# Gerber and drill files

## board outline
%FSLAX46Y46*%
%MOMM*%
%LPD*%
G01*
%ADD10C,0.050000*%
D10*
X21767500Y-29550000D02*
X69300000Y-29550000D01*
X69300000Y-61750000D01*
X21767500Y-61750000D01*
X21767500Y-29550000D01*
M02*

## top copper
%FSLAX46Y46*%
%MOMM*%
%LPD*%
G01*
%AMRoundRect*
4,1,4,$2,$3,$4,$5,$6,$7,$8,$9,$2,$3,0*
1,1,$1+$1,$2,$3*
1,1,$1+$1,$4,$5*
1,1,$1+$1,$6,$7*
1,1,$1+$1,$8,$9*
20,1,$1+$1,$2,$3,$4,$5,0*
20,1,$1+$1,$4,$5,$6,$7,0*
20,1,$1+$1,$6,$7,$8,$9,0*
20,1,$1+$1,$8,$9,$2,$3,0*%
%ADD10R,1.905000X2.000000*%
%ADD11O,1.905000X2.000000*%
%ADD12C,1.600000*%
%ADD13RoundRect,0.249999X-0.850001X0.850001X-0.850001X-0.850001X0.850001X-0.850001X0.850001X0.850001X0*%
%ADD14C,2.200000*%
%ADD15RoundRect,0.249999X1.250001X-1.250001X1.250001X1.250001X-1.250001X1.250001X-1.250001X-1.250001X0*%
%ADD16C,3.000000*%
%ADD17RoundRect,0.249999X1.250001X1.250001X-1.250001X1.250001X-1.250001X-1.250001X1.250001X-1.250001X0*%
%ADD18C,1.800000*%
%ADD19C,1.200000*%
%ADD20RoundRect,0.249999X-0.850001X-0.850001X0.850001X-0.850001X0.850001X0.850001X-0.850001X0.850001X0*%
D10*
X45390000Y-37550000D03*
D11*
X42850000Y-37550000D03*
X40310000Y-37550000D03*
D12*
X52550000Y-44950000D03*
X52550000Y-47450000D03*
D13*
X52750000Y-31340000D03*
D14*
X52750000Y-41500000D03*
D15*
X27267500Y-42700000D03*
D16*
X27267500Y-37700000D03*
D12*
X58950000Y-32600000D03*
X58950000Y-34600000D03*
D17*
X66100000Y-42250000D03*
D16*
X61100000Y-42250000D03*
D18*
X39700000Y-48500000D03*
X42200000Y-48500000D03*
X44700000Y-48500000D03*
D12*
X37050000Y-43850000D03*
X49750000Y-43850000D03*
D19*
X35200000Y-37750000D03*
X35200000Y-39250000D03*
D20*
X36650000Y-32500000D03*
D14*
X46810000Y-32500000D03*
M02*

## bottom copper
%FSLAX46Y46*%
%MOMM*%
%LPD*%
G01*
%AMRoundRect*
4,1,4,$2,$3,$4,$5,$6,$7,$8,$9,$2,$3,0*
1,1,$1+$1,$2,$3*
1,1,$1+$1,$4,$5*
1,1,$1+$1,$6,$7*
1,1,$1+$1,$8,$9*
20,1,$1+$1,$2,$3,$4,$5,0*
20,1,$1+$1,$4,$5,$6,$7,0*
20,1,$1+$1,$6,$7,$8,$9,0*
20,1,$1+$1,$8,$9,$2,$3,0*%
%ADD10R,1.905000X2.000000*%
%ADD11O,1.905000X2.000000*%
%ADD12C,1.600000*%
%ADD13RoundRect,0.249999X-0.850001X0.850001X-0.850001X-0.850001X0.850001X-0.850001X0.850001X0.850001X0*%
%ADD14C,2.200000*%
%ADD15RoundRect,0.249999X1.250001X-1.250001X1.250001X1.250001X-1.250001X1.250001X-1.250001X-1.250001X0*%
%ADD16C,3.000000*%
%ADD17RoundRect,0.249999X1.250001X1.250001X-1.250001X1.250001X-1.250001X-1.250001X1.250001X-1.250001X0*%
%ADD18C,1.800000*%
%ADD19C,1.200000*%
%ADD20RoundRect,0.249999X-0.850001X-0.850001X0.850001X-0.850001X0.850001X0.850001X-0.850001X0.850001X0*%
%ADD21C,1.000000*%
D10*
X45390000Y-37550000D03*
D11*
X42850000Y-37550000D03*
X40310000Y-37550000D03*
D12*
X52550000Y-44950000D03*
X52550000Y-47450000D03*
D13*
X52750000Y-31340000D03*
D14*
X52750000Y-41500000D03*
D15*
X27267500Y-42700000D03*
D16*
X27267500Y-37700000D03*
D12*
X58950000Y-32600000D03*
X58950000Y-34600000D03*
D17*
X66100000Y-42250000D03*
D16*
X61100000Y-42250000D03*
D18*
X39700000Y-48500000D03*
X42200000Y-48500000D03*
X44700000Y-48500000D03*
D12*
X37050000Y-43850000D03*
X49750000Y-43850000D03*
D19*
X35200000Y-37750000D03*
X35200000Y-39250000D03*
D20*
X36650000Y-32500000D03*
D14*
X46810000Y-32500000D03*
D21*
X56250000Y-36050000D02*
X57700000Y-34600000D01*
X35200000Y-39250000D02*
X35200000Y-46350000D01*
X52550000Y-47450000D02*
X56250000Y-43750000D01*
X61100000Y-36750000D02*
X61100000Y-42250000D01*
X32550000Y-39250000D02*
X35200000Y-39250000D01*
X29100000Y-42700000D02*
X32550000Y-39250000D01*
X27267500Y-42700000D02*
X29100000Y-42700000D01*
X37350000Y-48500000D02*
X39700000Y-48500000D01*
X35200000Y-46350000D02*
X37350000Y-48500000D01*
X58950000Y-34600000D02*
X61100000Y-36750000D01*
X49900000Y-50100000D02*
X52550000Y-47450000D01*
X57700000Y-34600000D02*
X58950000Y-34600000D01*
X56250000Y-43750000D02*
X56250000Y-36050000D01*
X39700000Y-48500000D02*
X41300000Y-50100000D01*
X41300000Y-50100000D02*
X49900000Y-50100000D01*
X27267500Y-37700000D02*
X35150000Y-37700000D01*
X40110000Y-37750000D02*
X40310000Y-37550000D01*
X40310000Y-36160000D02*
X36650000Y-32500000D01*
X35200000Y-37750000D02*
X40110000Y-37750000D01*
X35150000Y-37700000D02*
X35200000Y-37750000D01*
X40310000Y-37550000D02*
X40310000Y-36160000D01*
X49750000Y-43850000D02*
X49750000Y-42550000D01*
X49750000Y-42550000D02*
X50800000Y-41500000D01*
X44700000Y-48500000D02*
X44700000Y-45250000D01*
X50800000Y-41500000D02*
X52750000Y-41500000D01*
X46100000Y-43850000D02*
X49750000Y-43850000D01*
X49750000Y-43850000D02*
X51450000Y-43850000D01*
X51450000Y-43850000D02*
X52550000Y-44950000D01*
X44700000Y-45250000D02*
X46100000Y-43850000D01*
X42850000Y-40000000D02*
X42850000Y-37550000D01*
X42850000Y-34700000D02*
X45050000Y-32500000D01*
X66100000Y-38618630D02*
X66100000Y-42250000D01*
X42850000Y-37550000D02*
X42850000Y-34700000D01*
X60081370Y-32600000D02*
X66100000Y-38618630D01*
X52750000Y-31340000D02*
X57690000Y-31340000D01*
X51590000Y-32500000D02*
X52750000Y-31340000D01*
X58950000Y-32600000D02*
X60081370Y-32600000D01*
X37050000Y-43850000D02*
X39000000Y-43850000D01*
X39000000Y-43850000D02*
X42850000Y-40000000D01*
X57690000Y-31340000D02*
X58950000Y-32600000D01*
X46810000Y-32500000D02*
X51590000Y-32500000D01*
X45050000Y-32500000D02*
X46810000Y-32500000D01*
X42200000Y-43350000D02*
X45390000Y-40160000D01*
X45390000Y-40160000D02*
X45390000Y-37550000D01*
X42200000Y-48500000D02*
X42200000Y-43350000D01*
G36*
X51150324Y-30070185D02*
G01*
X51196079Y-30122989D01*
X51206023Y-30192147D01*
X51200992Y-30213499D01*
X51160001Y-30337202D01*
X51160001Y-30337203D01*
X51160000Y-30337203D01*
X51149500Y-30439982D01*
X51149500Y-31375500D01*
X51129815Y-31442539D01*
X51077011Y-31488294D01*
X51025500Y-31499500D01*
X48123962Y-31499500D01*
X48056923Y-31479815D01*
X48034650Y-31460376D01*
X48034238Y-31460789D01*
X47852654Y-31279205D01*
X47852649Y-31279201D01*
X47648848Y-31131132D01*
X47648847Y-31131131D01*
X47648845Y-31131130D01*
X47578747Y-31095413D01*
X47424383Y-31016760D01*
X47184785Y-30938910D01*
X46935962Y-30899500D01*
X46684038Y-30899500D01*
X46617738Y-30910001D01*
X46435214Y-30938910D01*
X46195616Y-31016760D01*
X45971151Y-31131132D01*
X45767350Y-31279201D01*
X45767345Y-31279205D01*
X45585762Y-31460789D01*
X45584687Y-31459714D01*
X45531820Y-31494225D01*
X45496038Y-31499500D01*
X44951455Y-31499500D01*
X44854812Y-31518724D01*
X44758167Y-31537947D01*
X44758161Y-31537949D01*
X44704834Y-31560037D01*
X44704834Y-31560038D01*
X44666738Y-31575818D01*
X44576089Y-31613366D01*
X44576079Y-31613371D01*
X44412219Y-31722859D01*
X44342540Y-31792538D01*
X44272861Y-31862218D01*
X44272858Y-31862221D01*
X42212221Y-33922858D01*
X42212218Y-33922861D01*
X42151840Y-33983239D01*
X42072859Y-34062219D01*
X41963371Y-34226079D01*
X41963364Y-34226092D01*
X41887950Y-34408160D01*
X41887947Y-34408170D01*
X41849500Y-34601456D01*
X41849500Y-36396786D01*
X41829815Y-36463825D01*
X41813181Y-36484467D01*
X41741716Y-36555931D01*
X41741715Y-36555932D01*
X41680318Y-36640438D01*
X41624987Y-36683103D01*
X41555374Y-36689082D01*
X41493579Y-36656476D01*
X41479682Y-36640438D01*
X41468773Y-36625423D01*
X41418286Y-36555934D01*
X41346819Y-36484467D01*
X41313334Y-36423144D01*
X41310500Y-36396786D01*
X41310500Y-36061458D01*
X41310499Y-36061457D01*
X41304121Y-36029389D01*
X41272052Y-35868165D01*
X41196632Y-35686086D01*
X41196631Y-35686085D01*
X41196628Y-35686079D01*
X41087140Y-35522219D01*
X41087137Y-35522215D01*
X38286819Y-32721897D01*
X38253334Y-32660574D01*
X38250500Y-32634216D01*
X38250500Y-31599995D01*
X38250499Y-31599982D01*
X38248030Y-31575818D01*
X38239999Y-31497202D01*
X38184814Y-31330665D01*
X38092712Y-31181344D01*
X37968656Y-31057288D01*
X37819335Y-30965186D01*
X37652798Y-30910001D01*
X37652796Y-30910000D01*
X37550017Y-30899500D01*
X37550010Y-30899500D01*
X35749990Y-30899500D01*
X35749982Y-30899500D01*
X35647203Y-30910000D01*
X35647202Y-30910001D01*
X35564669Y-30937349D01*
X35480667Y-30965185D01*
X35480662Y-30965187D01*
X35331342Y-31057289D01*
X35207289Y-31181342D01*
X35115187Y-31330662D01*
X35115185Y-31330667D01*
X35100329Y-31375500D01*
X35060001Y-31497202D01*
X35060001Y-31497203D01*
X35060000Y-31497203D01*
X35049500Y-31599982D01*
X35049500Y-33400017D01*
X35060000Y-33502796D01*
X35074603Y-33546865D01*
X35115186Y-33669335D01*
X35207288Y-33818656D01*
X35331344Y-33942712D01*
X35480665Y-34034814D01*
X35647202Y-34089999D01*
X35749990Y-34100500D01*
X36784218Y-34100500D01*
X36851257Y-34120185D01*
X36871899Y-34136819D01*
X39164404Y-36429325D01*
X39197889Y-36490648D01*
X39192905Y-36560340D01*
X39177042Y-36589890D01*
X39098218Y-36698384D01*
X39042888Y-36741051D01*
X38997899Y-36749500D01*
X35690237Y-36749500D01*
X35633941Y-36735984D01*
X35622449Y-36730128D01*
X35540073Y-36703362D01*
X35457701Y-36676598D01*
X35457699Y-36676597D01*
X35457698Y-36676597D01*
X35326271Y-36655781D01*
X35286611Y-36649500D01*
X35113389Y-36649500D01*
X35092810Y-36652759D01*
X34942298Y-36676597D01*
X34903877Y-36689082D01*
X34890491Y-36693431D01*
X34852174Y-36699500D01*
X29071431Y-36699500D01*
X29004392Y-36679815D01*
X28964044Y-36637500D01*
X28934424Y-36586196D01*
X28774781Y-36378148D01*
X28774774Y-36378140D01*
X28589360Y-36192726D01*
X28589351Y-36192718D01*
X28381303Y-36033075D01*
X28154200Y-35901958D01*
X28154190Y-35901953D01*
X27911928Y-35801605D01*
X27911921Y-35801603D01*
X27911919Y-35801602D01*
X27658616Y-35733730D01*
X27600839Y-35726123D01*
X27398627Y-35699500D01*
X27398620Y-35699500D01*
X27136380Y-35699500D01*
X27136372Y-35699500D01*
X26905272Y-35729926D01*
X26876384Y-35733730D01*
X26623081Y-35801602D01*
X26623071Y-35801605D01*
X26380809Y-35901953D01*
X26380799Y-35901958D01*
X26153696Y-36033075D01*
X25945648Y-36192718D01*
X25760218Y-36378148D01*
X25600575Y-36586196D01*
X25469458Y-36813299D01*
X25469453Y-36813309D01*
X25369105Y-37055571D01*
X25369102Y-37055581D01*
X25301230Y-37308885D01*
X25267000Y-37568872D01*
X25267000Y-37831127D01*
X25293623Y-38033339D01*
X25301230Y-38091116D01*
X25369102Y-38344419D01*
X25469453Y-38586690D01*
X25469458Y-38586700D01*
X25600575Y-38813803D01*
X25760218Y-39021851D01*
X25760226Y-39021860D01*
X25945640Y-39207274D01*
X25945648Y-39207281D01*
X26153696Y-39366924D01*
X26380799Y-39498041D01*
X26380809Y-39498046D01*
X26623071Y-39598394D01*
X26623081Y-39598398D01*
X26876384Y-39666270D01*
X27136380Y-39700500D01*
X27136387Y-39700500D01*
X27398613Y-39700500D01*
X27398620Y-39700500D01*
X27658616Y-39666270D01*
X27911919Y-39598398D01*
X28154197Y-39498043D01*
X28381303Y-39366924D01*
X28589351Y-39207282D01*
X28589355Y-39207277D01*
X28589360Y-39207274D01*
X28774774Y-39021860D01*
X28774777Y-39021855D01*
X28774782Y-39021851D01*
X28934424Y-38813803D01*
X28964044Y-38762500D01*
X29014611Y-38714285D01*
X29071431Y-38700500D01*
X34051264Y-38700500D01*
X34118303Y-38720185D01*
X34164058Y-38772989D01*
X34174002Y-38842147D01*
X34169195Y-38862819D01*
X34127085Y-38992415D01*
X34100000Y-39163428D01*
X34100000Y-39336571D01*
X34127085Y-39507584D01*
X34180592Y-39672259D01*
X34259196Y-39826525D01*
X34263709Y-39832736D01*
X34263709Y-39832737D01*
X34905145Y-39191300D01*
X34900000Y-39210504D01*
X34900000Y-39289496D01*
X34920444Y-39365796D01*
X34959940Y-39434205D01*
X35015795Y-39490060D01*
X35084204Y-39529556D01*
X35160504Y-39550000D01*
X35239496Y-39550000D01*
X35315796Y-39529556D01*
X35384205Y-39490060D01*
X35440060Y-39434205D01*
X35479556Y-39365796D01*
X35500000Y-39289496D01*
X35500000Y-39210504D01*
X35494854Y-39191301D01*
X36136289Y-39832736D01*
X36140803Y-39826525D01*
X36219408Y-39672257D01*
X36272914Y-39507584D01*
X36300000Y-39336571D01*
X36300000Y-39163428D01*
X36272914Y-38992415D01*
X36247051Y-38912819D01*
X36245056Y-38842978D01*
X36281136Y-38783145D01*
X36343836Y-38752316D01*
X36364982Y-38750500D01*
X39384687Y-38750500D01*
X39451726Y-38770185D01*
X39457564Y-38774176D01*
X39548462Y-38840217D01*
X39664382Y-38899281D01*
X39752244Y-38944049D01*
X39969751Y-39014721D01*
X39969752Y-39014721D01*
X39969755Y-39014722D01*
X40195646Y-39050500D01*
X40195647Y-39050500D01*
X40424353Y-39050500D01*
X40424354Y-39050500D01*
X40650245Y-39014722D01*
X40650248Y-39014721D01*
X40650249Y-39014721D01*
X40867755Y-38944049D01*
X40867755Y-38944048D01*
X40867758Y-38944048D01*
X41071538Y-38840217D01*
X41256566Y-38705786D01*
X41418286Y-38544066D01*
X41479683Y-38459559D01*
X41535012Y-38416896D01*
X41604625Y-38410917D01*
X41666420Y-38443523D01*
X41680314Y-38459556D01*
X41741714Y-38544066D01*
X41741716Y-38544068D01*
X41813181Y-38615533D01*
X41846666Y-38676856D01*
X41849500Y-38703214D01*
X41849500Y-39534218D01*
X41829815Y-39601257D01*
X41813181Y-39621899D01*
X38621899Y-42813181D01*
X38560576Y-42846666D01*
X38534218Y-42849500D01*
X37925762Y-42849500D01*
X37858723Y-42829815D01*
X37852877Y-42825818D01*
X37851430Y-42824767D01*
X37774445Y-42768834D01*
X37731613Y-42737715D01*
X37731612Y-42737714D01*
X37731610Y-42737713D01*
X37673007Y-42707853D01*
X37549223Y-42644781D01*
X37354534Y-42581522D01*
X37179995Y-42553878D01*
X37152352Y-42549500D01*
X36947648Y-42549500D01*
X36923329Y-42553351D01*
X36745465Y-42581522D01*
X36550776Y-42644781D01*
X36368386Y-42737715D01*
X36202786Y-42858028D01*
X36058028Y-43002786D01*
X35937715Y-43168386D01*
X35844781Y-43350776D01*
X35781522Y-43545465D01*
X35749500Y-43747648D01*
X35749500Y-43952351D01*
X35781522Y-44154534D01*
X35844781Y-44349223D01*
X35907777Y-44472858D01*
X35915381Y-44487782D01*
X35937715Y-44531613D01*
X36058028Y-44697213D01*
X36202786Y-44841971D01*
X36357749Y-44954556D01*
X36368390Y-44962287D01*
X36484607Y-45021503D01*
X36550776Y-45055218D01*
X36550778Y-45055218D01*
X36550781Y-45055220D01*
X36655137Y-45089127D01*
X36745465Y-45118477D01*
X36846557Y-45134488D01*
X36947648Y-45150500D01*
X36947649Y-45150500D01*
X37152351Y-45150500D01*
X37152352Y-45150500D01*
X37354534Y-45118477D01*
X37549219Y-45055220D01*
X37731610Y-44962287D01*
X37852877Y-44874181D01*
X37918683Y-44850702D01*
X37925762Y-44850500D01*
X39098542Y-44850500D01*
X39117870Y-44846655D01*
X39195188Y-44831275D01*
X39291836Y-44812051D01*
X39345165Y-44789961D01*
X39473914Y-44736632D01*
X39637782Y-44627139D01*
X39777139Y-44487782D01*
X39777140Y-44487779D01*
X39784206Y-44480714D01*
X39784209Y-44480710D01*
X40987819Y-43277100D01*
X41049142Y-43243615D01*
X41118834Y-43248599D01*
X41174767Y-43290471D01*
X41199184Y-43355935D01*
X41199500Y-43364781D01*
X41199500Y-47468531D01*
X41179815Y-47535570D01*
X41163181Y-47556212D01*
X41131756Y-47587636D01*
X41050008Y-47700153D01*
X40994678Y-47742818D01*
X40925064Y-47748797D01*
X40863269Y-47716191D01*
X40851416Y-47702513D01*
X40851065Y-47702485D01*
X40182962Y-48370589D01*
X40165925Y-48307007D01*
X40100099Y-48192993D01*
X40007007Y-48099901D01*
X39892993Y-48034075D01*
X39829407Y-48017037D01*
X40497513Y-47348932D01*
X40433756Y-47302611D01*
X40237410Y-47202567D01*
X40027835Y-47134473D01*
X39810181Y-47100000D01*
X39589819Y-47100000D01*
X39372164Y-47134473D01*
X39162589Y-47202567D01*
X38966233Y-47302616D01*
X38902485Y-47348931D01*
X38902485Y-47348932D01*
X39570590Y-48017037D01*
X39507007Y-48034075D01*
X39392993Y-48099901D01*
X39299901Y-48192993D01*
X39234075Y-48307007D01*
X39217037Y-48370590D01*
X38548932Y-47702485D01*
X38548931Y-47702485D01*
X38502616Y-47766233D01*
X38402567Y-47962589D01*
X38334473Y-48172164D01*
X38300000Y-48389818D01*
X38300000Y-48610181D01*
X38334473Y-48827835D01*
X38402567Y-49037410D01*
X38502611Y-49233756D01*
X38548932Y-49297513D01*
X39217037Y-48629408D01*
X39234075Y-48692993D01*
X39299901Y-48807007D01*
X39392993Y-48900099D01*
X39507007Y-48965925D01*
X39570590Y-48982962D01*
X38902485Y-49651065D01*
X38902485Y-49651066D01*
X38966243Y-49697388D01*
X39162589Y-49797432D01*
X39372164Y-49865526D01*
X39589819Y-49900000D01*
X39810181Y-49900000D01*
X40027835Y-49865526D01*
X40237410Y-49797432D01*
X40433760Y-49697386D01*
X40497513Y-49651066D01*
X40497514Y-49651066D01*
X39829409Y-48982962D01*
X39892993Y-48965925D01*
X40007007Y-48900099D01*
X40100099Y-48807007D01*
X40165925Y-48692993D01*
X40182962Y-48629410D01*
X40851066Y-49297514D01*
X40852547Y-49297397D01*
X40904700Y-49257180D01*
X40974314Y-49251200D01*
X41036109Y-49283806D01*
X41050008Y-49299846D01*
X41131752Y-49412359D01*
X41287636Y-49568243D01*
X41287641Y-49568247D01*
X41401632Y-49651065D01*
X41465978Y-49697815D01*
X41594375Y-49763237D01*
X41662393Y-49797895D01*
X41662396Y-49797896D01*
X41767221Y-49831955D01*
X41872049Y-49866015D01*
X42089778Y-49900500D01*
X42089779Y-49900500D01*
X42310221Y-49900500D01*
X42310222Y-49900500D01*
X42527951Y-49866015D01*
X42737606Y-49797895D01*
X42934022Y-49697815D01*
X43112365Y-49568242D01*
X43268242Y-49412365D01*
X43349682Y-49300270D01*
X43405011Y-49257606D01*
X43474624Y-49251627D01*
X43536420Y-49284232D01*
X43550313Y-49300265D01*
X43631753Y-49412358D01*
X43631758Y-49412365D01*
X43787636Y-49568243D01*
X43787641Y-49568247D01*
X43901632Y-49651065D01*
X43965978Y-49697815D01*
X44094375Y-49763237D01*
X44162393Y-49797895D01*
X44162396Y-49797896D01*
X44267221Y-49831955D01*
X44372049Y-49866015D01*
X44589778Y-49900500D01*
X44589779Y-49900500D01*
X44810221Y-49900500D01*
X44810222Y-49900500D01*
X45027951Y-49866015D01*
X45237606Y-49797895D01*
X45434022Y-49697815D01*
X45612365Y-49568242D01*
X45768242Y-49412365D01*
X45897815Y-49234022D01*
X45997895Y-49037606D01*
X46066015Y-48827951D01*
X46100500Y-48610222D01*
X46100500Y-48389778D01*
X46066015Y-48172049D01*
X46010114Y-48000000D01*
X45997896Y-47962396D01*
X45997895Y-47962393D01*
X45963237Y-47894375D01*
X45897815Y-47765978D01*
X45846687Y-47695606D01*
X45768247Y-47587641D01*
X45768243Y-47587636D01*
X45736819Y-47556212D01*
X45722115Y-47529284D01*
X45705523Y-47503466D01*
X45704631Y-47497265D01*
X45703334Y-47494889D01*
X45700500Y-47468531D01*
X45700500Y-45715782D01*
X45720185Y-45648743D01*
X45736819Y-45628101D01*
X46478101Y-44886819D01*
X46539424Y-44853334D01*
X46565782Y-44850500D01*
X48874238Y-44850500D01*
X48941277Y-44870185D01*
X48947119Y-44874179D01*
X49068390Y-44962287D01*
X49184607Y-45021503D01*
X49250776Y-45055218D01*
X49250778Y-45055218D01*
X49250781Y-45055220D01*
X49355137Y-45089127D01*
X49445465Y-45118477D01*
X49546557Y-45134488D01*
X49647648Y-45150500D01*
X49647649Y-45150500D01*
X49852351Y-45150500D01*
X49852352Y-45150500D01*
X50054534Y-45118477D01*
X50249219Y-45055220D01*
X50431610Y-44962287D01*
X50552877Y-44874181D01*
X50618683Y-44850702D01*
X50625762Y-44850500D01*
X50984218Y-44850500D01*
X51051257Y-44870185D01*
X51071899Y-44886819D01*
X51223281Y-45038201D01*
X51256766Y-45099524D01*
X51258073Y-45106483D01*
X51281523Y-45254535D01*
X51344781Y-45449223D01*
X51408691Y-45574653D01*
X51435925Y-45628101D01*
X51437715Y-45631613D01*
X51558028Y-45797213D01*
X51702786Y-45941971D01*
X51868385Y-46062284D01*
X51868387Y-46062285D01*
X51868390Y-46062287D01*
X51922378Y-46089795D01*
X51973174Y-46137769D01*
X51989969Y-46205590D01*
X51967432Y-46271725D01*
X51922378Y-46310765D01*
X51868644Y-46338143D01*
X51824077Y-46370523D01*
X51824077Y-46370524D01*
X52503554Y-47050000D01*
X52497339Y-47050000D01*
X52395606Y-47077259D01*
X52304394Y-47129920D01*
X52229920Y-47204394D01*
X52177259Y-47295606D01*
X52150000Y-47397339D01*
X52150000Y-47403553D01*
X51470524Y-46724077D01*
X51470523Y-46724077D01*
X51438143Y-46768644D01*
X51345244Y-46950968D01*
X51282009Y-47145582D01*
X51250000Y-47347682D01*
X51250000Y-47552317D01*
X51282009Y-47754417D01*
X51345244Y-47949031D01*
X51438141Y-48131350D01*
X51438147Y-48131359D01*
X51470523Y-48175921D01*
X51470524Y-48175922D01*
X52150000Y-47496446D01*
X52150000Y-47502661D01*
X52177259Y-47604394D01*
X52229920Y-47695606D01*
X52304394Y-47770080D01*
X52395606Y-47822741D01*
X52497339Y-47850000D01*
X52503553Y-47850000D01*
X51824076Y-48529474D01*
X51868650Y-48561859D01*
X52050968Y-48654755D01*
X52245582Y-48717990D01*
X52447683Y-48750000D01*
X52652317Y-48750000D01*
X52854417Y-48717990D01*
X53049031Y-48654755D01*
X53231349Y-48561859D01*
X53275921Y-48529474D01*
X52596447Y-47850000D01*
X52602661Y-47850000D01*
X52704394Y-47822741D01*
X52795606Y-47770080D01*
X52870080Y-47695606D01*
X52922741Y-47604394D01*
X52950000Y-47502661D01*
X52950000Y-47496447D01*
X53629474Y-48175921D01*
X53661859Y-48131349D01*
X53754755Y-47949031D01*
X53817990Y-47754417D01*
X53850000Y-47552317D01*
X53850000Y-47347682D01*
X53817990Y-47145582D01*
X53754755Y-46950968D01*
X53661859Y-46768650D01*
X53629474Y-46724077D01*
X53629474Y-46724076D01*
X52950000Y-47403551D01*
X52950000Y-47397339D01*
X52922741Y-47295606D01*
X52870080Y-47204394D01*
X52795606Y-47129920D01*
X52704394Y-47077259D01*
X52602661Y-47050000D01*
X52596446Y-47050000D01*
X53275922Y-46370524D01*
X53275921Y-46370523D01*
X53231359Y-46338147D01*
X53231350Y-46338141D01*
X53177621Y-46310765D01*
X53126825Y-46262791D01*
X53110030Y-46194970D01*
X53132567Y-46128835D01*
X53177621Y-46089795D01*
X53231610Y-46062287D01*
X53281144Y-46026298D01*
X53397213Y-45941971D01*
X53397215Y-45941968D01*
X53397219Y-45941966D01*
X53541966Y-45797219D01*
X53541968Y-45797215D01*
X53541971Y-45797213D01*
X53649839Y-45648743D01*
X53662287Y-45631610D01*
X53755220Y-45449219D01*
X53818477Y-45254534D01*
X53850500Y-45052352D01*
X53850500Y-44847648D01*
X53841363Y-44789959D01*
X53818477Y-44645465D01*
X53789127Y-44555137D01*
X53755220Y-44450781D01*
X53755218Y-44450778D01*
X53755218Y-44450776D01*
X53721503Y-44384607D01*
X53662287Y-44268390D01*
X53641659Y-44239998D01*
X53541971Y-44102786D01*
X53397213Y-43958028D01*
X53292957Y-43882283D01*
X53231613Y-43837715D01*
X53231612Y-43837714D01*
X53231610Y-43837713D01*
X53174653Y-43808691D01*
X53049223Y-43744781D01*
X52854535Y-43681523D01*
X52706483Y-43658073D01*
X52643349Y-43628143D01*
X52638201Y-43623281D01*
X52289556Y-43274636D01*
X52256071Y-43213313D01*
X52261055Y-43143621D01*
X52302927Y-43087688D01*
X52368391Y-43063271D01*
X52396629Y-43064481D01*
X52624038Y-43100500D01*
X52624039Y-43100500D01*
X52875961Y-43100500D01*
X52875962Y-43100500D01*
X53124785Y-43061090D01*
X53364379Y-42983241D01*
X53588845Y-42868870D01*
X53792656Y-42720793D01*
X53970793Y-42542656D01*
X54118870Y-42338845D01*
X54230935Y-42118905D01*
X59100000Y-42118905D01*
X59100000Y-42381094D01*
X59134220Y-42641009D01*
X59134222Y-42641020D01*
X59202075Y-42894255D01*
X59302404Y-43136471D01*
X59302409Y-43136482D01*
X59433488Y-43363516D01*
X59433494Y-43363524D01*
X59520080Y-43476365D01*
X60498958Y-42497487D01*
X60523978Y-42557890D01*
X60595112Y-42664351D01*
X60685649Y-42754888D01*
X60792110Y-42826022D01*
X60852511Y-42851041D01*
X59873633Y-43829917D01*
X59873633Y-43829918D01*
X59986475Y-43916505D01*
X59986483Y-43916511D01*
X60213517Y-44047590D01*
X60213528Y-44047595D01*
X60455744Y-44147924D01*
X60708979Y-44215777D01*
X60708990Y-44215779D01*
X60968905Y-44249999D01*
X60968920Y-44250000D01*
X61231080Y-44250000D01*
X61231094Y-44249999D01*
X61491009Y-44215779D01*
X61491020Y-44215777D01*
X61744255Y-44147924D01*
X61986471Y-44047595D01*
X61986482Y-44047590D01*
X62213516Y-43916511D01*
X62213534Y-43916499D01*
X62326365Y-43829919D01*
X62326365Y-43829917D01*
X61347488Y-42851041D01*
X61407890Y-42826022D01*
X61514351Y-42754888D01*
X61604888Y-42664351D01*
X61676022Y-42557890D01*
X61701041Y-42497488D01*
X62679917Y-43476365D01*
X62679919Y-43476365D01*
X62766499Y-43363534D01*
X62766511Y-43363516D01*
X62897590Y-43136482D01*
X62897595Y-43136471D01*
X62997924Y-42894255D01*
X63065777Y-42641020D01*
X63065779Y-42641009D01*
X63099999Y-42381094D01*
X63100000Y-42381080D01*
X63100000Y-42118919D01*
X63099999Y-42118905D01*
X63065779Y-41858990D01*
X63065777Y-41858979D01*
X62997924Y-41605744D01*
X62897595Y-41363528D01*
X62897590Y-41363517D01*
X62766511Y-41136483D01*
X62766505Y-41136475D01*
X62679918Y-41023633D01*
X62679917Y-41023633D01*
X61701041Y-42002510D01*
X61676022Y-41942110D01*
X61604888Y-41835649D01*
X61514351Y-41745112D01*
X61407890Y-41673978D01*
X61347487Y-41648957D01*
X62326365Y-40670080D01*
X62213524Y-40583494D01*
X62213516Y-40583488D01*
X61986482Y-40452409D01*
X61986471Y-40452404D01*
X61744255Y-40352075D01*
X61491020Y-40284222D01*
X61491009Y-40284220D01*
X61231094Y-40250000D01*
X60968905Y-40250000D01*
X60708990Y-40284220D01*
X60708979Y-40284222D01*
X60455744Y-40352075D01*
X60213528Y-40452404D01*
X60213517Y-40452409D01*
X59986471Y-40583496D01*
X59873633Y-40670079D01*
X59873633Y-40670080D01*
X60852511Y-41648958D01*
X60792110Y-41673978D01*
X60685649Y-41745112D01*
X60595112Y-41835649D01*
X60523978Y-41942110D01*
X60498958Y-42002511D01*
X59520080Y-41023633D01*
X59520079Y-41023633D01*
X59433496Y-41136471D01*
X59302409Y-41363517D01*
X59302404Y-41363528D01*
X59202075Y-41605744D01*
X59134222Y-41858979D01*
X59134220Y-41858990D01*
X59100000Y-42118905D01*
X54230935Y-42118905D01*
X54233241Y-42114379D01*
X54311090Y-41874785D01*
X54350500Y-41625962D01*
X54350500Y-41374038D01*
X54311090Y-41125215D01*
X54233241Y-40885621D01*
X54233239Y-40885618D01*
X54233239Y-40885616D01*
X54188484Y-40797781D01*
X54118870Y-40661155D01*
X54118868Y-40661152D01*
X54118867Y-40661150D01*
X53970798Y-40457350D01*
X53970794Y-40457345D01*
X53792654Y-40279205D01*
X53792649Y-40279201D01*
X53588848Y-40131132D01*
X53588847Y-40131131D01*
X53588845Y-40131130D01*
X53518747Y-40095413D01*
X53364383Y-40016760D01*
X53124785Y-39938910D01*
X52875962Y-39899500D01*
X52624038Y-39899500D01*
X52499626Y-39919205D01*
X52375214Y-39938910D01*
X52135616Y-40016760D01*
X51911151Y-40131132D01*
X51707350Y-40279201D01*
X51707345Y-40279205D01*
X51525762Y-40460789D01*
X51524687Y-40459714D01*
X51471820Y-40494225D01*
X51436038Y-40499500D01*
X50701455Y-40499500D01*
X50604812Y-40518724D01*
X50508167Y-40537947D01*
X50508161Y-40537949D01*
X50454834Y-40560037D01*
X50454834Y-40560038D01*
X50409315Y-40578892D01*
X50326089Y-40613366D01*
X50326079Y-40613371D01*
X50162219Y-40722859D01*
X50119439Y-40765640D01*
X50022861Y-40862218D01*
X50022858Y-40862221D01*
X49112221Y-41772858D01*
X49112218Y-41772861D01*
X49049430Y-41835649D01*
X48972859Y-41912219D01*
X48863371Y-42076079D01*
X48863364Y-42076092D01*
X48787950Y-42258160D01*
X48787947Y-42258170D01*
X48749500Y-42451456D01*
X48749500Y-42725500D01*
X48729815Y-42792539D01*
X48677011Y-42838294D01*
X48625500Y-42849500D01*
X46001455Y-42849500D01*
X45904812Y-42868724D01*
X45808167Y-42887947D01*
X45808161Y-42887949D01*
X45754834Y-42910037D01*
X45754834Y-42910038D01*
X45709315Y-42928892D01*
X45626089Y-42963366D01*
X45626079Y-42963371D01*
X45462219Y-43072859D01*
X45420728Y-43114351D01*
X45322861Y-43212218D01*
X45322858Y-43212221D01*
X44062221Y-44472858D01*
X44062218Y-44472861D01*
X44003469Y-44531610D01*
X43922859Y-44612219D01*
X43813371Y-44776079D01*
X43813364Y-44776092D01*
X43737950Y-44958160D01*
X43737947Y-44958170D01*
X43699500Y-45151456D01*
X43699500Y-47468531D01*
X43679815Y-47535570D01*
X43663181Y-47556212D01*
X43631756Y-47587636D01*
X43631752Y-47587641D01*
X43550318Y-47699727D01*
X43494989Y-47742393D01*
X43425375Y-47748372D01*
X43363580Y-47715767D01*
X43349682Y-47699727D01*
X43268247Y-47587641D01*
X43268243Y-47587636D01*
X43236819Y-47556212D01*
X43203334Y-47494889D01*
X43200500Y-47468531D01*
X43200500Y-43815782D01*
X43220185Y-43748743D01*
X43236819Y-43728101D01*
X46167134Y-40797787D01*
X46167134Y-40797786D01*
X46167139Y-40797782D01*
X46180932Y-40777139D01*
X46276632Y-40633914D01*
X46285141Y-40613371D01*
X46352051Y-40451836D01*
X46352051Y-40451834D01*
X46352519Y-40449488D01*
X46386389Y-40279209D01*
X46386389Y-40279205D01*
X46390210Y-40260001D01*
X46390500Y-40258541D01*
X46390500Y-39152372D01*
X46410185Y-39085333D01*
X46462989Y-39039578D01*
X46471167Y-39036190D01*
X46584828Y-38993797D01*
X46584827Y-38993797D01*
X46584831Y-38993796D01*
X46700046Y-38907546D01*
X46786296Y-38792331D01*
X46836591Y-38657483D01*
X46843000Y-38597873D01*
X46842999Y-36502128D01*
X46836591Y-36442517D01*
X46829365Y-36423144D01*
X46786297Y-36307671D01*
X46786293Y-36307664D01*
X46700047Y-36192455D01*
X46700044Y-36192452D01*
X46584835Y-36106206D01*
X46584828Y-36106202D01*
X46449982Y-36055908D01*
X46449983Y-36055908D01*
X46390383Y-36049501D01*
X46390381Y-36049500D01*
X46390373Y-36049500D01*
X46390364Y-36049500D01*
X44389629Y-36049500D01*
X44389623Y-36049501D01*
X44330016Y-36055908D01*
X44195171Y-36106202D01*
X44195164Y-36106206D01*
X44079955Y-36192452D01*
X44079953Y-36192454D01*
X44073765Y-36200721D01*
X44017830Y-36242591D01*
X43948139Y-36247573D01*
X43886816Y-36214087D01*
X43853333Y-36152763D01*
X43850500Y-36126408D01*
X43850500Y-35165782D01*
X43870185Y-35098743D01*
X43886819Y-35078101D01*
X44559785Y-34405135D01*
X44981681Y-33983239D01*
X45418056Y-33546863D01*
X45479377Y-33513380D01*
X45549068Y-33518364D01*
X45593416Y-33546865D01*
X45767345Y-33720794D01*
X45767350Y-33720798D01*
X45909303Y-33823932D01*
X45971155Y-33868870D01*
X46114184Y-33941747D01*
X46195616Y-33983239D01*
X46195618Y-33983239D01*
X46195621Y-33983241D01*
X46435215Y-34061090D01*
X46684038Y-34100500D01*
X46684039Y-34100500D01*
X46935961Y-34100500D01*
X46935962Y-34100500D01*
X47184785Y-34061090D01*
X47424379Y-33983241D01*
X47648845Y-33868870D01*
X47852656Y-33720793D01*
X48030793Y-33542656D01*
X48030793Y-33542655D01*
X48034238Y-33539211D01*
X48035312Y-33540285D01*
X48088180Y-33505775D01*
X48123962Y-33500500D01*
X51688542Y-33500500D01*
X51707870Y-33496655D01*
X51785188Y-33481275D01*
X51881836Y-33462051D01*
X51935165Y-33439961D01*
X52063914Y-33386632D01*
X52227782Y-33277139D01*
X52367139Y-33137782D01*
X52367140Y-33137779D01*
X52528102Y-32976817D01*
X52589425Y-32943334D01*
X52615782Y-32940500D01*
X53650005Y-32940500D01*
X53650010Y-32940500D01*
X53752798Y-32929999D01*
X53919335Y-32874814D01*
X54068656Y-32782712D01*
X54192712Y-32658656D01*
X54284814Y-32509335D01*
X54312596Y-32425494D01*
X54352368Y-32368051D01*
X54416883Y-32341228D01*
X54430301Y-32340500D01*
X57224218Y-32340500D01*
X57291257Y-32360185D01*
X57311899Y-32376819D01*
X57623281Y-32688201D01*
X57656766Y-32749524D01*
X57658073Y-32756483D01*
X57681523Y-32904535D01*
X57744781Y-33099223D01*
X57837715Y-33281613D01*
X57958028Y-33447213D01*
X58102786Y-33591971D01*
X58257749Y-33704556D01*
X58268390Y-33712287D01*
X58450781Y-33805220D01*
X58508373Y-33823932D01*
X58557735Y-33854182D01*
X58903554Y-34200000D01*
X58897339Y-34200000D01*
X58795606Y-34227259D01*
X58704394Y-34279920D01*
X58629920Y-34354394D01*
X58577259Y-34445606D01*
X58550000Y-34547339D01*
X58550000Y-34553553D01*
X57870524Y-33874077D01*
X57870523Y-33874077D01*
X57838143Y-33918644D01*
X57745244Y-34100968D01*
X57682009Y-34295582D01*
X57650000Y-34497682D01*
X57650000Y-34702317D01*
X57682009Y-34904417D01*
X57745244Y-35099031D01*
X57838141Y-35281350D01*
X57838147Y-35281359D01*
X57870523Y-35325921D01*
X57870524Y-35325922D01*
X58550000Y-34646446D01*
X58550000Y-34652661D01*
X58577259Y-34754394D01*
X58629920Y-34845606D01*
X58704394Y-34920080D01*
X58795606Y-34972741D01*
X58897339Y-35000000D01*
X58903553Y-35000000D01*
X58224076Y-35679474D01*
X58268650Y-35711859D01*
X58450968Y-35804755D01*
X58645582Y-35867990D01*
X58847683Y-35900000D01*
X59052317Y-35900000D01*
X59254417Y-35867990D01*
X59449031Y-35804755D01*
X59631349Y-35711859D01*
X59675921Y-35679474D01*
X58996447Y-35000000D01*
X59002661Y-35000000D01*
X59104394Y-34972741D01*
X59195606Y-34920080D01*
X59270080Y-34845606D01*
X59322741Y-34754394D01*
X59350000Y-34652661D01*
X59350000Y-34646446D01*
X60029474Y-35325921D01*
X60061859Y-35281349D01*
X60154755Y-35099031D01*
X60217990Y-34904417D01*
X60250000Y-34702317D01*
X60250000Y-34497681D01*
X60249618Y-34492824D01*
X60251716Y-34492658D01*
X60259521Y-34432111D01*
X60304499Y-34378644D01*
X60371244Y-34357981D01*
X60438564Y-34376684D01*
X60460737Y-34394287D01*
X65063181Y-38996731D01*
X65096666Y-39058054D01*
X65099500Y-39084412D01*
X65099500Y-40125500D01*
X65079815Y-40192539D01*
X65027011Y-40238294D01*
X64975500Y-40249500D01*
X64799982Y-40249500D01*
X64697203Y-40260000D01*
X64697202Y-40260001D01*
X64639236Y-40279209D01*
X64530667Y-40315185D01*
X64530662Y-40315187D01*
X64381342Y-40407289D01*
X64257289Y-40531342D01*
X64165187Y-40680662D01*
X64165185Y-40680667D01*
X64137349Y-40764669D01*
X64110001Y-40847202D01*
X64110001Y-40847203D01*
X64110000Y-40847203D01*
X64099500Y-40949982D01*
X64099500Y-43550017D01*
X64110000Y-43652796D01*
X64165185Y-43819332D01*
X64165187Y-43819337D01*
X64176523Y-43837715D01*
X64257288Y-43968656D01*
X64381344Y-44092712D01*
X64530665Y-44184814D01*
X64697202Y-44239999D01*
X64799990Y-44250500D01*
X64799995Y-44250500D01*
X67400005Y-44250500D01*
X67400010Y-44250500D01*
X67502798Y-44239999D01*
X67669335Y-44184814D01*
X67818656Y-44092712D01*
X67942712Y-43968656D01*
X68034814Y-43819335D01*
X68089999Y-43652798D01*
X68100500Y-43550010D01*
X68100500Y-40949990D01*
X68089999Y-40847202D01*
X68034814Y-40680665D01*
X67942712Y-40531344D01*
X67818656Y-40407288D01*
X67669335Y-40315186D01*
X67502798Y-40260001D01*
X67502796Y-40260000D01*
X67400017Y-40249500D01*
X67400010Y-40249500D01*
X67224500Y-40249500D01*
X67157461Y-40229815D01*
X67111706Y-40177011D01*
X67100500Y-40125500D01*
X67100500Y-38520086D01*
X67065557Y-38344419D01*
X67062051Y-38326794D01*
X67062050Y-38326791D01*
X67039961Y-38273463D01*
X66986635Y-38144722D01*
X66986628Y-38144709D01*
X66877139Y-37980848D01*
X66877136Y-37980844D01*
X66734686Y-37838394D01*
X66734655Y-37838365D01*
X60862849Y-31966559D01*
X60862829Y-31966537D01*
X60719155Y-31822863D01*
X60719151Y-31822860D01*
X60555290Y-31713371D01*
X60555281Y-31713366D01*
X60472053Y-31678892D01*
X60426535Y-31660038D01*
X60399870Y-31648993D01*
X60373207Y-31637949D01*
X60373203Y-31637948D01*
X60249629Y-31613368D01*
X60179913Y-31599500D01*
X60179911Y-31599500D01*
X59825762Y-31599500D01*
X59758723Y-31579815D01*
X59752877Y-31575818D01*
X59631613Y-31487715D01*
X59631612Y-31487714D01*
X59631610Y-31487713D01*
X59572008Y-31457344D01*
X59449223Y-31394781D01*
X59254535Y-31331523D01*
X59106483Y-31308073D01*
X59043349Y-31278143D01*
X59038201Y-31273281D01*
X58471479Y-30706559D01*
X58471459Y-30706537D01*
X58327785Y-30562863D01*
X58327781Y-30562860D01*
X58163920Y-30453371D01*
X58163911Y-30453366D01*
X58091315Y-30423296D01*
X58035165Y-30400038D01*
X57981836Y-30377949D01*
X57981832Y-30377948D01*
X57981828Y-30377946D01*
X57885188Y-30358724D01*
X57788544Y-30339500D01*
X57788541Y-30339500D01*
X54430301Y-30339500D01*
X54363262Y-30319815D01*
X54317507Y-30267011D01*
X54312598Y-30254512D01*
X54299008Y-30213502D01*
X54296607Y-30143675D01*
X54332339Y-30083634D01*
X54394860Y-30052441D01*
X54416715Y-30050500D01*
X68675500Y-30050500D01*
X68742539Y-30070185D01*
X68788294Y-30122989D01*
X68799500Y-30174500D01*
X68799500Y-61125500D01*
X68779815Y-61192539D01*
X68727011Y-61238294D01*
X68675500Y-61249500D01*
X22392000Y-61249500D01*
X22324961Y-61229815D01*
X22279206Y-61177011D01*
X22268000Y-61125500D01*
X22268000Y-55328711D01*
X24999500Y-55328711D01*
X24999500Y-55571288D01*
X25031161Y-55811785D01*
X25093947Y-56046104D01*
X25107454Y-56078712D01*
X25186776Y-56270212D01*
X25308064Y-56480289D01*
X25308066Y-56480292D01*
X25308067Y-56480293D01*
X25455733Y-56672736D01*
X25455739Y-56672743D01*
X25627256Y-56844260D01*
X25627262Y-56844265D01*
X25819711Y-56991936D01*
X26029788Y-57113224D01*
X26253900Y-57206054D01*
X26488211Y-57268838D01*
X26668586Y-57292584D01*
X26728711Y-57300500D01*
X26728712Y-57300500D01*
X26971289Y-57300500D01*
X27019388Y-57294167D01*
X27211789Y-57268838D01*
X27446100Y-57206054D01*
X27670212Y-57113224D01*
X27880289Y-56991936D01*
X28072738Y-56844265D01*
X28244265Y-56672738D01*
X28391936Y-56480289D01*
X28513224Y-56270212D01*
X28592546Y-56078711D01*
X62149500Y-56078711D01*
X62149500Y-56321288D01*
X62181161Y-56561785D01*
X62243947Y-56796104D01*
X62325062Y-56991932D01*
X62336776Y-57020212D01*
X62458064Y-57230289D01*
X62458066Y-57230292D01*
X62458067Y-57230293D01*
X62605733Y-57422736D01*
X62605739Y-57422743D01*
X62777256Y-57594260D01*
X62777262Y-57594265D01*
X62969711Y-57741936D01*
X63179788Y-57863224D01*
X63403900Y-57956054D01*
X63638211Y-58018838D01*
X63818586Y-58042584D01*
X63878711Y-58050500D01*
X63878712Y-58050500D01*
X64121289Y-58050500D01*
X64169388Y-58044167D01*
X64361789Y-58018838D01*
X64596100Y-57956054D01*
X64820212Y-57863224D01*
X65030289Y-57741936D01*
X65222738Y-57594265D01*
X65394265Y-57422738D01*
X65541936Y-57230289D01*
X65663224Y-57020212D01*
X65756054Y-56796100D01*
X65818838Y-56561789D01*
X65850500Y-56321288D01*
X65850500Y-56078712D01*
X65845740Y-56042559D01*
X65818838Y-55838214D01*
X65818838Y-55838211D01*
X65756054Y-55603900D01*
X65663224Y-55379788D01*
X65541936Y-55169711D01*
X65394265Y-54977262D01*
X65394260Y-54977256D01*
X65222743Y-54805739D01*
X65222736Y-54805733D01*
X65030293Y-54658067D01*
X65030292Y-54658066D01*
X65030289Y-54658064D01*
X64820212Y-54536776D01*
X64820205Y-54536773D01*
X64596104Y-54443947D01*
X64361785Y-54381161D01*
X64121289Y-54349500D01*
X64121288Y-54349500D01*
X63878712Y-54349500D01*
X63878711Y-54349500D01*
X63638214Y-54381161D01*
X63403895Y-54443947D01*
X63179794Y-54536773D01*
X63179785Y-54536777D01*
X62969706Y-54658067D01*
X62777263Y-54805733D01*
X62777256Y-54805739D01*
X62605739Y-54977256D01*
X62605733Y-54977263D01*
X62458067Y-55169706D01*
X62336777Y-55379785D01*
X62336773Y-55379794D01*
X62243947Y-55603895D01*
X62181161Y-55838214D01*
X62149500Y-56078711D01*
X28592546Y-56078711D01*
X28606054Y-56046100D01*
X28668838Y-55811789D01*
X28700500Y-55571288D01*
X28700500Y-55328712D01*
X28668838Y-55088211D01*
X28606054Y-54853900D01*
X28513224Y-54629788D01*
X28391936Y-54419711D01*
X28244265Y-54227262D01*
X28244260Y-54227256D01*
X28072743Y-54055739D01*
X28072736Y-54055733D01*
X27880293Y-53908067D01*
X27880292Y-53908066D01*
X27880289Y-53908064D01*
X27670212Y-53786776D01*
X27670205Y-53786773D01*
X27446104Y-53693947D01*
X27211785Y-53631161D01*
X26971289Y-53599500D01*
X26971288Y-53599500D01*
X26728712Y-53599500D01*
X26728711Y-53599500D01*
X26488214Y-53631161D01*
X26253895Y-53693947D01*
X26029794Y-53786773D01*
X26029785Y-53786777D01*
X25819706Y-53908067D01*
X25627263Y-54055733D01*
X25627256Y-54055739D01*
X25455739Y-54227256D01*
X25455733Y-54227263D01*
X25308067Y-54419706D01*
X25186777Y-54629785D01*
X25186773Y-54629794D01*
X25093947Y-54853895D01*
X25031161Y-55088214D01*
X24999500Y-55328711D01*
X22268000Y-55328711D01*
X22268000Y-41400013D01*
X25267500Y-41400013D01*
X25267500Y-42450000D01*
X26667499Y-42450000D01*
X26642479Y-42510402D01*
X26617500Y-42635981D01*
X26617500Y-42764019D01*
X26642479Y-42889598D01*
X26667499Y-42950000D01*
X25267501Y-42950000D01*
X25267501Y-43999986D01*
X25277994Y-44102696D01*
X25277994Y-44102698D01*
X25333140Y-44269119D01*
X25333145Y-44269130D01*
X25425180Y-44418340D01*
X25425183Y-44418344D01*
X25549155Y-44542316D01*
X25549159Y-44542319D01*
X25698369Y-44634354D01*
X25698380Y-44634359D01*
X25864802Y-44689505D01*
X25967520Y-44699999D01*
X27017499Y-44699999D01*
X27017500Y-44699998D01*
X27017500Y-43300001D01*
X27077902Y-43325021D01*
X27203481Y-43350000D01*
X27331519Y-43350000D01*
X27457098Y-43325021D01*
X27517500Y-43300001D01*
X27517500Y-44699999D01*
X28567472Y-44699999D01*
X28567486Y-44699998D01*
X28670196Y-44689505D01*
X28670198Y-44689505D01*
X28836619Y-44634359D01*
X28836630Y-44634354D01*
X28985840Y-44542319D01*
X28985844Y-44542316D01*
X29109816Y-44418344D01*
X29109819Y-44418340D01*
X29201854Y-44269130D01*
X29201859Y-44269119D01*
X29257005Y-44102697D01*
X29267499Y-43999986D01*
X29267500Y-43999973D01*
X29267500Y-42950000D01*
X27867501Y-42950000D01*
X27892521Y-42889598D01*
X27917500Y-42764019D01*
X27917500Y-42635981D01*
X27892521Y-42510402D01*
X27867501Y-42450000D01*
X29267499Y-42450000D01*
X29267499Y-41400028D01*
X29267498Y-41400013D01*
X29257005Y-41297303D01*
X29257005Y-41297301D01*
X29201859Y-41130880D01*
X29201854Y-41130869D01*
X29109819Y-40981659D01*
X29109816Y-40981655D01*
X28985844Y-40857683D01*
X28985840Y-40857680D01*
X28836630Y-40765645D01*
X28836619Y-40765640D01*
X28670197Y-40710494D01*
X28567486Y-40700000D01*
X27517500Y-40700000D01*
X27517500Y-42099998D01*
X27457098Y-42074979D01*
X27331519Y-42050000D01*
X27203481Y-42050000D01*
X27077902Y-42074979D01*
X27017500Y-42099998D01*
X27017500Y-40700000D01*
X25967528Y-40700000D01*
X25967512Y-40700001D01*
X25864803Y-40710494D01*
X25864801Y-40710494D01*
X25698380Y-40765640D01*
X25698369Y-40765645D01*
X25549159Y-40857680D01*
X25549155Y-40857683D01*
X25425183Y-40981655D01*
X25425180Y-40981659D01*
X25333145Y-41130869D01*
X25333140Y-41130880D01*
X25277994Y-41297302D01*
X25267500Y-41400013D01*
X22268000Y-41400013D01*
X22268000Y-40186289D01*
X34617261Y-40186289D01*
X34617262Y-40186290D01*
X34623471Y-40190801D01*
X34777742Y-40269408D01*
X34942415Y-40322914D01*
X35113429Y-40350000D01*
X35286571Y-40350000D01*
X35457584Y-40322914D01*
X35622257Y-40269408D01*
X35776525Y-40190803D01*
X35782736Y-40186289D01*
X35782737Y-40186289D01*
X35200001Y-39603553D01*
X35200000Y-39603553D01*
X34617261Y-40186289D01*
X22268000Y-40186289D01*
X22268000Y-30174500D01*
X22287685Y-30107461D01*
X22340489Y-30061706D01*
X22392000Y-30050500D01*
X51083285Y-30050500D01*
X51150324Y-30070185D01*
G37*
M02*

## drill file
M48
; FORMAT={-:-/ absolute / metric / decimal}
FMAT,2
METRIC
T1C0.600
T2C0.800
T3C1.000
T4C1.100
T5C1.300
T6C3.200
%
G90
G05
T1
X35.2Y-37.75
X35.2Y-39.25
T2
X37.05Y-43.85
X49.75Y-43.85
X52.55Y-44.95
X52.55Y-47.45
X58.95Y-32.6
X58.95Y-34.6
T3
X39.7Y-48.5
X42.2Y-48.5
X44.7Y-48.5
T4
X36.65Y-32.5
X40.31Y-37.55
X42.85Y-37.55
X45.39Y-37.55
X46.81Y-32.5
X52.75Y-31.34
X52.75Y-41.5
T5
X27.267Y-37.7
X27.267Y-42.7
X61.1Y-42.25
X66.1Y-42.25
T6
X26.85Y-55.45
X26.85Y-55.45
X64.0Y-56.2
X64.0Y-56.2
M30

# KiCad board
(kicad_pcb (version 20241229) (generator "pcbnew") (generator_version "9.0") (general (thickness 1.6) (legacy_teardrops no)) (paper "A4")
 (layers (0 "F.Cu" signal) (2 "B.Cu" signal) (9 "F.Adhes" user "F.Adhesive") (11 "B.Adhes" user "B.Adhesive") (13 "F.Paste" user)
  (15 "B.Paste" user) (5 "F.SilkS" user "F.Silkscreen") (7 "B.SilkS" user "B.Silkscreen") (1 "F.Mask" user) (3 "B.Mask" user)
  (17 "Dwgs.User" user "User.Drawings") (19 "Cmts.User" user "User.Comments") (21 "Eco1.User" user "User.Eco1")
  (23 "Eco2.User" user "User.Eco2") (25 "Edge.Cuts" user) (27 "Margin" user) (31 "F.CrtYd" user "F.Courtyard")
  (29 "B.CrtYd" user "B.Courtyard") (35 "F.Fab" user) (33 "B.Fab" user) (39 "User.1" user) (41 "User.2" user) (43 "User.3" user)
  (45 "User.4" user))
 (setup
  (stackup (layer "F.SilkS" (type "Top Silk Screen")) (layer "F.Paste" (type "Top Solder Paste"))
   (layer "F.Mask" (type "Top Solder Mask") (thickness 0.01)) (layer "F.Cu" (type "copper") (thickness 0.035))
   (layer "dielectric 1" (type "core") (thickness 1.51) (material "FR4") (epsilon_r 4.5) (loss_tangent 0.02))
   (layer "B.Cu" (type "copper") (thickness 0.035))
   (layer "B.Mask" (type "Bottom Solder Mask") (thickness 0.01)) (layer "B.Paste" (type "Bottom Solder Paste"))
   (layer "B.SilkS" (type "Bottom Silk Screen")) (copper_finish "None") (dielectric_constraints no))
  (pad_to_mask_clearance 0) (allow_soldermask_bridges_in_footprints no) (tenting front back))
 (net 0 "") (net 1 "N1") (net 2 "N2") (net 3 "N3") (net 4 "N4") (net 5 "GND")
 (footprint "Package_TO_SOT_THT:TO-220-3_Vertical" (layer "F.Cu") (at 45.39 37.55 180)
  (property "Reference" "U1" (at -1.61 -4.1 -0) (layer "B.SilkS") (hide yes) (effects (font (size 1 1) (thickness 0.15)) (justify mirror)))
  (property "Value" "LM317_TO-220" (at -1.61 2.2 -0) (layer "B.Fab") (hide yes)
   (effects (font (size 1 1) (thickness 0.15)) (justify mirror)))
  (pad "1" thru_hole rect (at 0 0 180) (size 1.905 2) (drill 1.1) (layers "*.Cu" "*.Mask") (remove_unused_layers no) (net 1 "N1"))
  (pad "2" thru_hole oval (at 2.54 0 180) (size 1.905 2) (drill 1.1) (layers "*.Cu" "*.Mask") (remove_unused_layers no) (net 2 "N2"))
  (pad "3" thru_hole oval (at 5.08 0 180) (size 1.905 2) (drill 1.1) (layers "*.Cu" "*.Mask") (remove_unused_layers no) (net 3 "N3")))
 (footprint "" (layer "F.Cu") (at 26.85 55.45)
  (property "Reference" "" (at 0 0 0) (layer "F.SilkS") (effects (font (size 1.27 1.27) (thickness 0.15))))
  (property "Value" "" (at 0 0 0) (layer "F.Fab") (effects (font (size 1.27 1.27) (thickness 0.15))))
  (pad "" np_thru_hole circle (at 0 0) (size 3.2 3.2) (drill 3.2) (layers "*.Cu" "*.Mask")))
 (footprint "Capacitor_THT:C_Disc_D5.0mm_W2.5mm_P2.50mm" (layer "F.Cu") (at 52.55 44.95 -90)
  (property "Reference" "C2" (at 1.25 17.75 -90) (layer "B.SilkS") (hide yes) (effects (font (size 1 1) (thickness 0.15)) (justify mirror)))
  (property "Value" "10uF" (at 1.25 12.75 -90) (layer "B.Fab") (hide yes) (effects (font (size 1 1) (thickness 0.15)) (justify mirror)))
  (pad "1" thru_hole circle (at 0 0 270) (size 1.6 1.6) (drill 0.8) (layers "*.Cu" "*.Mask") (remove_unused_layers no) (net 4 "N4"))
  (pad "2" thru_hole circle (at 2.5 0 270) (size 1.6 1.6) (drill 0.8) (layers "*.Cu" "*.Mask") (remove_unused_layers no) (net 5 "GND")))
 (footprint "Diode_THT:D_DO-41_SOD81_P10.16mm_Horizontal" (layer "F.Cu") (at 52.75 31.34 -90)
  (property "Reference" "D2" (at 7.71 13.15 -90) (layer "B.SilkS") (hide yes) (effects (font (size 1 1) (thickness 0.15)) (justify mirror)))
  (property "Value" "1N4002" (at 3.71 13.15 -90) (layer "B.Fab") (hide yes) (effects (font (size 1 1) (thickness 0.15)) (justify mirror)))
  (pad "1" thru_hole roundrect (at 0 0 270) (size 2.2 2.2) (drill 1.1) (layers "*.Cu" "*.Mask") (remove_unused_layers no)
   (roundrect_rratio 0.113636) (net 2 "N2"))
  (pad "2" thru_hole circle (at 10.16 0 270) (size 2.2 2.2) (drill 1.1) (layers "*.Cu" "*.Mask") (remove_unused_layers no) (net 4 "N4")))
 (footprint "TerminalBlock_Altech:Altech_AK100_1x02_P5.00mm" (layer "F.Cu") (at 27.2675 42.7 90)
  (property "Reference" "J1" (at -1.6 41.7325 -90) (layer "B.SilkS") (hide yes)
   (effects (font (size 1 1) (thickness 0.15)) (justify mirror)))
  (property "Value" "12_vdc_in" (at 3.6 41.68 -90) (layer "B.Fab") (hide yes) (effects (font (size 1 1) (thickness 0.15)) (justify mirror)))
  (pad "1" thru_hole roundrect (at 0 0 90) (size 3 3) (drill 1.3) (layers "*.Cu" "*.Mask") (remove_unused_layers no)
   (roundrect_rratio 0.083333) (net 5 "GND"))
  (pad "2" thru_hole circle (at 5 0 90) (size 3 3) (drill 1.3) (layers "*.Cu" "*.Mask") (remove_unused_layers no) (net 3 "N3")))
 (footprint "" (layer "F.Cu") (at 64 56.2)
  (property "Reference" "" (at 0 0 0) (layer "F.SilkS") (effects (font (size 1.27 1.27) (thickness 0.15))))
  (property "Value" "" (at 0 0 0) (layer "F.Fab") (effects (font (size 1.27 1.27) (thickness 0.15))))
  (pad "" np_thru_hole circle (at 0 0) (size 3.2 3.2) (drill 3.2) (layers "*.Cu" "*.Mask")))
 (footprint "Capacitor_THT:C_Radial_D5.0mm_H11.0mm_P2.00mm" (layer "F.Cu") (at 58.95 32.6 -90)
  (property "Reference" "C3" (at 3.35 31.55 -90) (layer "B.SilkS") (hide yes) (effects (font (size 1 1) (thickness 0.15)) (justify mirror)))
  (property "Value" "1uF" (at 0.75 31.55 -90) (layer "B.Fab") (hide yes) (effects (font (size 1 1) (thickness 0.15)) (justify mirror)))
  (pad "1" thru_hole circle (at 0 0 270) (size 1.6 1.6) (drill 0.8) (layers "*.Cu" "*.Mask") (remove_unused_layers no) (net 2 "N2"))
  (pad "2" thru_hole circle (at 2 0 270) (size 1.6 1.6) (drill 0.8) (layers "*.Cu" "*.Mask") (remove_unused_layers no) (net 5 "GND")))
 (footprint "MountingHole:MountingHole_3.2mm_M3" (layer "F.Cu") (at 64 56.2)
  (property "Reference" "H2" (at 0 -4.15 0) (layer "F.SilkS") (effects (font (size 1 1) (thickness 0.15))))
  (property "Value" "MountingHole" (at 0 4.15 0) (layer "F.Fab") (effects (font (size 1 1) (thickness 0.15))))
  (pad "" np_thru_hole circle (at 0 0) (size 3.2 3.2) (drill 3.2) (layers "*.Cu" "*.Mask")))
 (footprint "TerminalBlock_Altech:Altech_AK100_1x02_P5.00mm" (layer "F.Cu") (at 66.1 42.25 180)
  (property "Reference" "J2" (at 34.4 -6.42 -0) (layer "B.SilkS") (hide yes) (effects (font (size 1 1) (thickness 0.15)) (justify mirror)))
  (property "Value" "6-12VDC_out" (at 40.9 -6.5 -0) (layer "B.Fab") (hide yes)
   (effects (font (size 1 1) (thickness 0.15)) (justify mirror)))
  (pad "1" thru_hole roundrect (at 0 0 180) (size 3 3) (drill 1.3) (layers "*.Cu" "*.Mask") (remove_unused_layers no)
   (roundrect_rratio 0.083333) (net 2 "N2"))
  (pad "2" thru_hole circle (at 5 0 180) (size 3 3) (drill 1.3) (layers "*.Cu" "*.Mask") (remove_unused_layers no) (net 5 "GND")))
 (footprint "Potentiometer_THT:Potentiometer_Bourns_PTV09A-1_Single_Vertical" (layer "F.Cu") (at 39.7 48.5 -90)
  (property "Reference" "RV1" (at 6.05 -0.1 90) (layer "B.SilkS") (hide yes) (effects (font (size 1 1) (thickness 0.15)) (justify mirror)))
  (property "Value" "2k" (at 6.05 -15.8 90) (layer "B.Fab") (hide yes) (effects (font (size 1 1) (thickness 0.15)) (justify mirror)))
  (pad "1" thru_hole circle (at 0 0 270) (size 1.8 1.8) (drill 1) (layers "*.Cu" "*.Mask") (remove_unused_layers no) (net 5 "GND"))
  (pad "2" thru_hole circle (at 0 -2.5 270) (size 1.8 1.8) (drill 1) (layers "*.Cu" "*.Mask") (remove_unused_layers no) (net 1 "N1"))
  (pad "3" thru_hole circle (at 0 -5 270) (size 1.8 1.8) (drill 1) (layers "*.Cu" "*.Mask") (remove_unused_layers no) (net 4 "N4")))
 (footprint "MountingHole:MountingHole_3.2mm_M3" (layer "F.Cu") (at 26.85 55.45)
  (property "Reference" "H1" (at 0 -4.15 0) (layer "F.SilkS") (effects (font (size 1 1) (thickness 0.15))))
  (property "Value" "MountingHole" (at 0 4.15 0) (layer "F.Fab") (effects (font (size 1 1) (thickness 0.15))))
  (pad "" np_thru_hole circle (at 0 0) (size 3.2 3.2) (drill 3.2) (layers "*.Cu" "*.Mask")))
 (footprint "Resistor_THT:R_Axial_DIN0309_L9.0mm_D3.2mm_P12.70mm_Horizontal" (layer "F.Cu") (at 37.05 43.85)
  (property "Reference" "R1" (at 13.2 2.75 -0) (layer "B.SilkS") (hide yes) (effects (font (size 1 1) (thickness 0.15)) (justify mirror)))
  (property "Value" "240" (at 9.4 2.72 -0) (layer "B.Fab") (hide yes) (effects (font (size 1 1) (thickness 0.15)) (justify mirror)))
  (pad "1" thru_hole circle (at 0 0) (size 1.6 1.6) (drill 0.8) (layers "*.Cu" "*.Mask") (remove_unused_layers no) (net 2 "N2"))
  (pad "2" thru_hole circle (at 12.7 0) (size 1.6 1.6) (drill 0.8) (layers "*.Cu" "*.Mask") (remove_unused_layers no) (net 4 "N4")))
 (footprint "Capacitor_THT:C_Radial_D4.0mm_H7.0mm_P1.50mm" (layer "F.Cu") (at 35.2 37.75 -90)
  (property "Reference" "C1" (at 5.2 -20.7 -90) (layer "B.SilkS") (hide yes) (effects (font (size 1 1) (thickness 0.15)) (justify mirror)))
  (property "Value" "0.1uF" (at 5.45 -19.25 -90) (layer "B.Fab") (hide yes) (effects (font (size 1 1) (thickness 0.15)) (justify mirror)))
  (pad "1" thru_hole circle (at 0 0 270) (size 1.2 1.2) (drill 0.6) (layers "*.Cu" "*.Mask") (remove_unused_layers no) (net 3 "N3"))
  (pad "2" thru_hole circle (at 1.5 0 270) (size 1.2 1.2) (drill 0.6) (layers "*.Cu" "*.Mask") (remove_unused_layers no) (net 5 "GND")))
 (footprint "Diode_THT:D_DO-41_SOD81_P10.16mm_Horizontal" (layer "F.Cu") (at 36.65 32.5)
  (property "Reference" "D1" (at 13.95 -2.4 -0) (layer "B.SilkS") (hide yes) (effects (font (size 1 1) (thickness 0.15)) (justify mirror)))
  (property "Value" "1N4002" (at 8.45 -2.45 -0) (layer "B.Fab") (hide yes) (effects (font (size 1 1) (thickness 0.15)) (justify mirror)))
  (pad "1" thru_hole roundrect (at 0 0) (size 2.2 2.2) (drill 1.1) (layers "*.Cu" "*.Mask") (remove_unused_layers no)
   (roundrect_rratio 0.113636) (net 3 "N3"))
  (pad "2" thru_hole circle (at 10.16 0) (size 2.2 2.2) (drill 1.1) (layers "*.Cu" "*.Mask") (remove_unused_layers no) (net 2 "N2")))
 (gr_rect (start 21.7675 29.55) (end 69.3 61.75) (stroke (width 0.05) (type default)) (fill no) (layer "Edge.Cuts"))
 (segment (start 56.25 36.05) (end 57.7 34.6) (width 1) (layer "B.Cu") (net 5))
 (segment (start 35.2 39.25) (end 35.2 46.35) (width 1) (layer "B.Cu") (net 5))
 (segment (start 52.55 47.45) (end 56.25 43.75) (width 1) (layer "B.Cu") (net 5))
 (segment (start 61.1 36.75) (end 61.1 42.25) (width 1) (layer "B.Cu") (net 5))
 (segment (start 32.55 39.25) (end 35.2 39.25) (width 1) (layer "B.Cu") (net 5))
 (segment (start 29.1 42.7) (end 32.55 39.25) (width 1) (layer "B.Cu") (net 5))
 (segment (start 27.2675 42.7) (end 29.1 42.7) (width 1) (layer "B.Cu") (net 5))
 (segment (start 37.35 48.5) (end 39.7 48.5) (width 1) (layer "B.Cu") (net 5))
 (segment (start 35.2 46.35) (end 37.35 48.5) (width 1) (layer "B.Cu") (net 5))
 (segment (start 58.95 34.6) (end 61.1 36.75) (width 1) (layer "B.Cu") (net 5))
 (segment (start 49.9 50.1) (end 52.55 47.45) (width 1) (layer "B.Cu") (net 5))
 (segment (start 57.7 34.6) (end 58.95 34.6) (width 1) (layer "B.Cu") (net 5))
 (segment (start 56.25 43.75) (end 56.25 36.05) (width 1) (layer "B.Cu") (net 5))
 (segment (start 39.7 48.5) (end 41.3 50.1) (width 1) (layer "B.Cu") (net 5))
 (segment (start 41.3 50.1) (end 49.9 50.1) (width 1) (layer "B.Cu") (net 5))
 (segment (start 27.2675 37.7) (end 35.15 37.7) (width 1) (layer "B.Cu") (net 3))
 (segment (start 40.11 37.75) (end 40.31 37.55) (width 1) (layer "B.Cu") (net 3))
 (segment (start 40.31 36.16) (end 36.65 32.5) (width 1) (layer "B.Cu") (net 3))
 (segment (start 35.2 37.75) (end 40.11 37.75) (width 1) (layer "B.Cu") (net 3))
 (segment (start 35.15 37.7) (end 35.2 37.75) (width 1) (layer "B.Cu") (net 3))
 (segment (start 40.31 37.55) (end 40.31 36.16) (width 1) (layer "B.Cu") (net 3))
 (segment (start 49.75 43.85) (end 49.75 42.55) (width 1) (layer "B.Cu") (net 4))
 (segment (start 49.75 42.55) (end 50.8 41.5) (width 1) (layer "B.Cu") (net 4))
 (segment (start 44.7 48.5) (end 44.7 45.25) (width 1) (layer "B.Cu") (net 4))
 (segment (start 50.8 41.5) (end 52.75 41.5) (width 1) (layer "B.Cu") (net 4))
 (segment (start 46.1 43.85) (end 49.75 43.85) (width 1) (layer "B.Cu") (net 4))
 (segment (start 49.75 43.85) (end 51.45 43.85) (width 1) (layer "B.Cu") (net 4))
 (segment (start 51.45 43.85) (end 52.55 44.95) (width 1) (layer "B.Cu") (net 4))
 (segment (start 44.7 45.25) (end 46.1 43.85) (width 1) (layer "B.Cu") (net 4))
 (segment (start 42.85 40) (end 42.85 37.55) (width 1) (layer "B.Cu") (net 2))
 (segment (start 42.85 34.7) (end 45.05 32.5) (width 1) (layer "B.Cu") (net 2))
 (segment (start 66.1 38.61863) (end 66.1 42.25) (width 1) (layer "B.Cu") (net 2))
 (segment (start 42.85 37.55) (end 42.85 34.7) (width 1) (layer "B.Cu") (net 2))
 (segment (start 60.08137 32.6) (end 66.1 38.61863) (width 1) (layer "B.Cu") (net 2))
 (segment (start 52.75 31.34) (end 57.69 31.34) (width 1) (layer "B.Cu") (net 2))
 (segment (start 51.59 32.5) (end 52.75 31.34) (width 1) (layer "B.Cu") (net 2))
 (segment (start 58.95 32.6) (end 60.08137 32.6) (width 1) (layer "B.Cu") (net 2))
 (segment (start 37.05 43.85) (end 39 43.85) (width 1) (layer "B.Cu") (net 2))
 (segment (start 39 43.85) (end 42.85 40) (width 1) (layer "B.Cu") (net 2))
 (segment (start 57.69 31.34) (end 58.95 32.6) (width 1) (layer "B.Cu") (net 2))
 (segment (start 46.81 32.5) (end 51.59 32.5) (width 1) (layer "B.Cu") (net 2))
 (segment (start 45.05 32.5) (end 46.81 32.5) (width 1) (layer "B.Cu") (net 2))
 (segment (start 42.2 43.35) (end 45.39 40.16) (width 1) (layer "B.Cu") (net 1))
 (segment (start 45.39 40.16) (end 45.39 37.55) (width 1) (layer "B.Cu") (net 1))
 (segment (start 42.2 48.5) (end 42.2 43.35) (width 1) (layer "B.Cu") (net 1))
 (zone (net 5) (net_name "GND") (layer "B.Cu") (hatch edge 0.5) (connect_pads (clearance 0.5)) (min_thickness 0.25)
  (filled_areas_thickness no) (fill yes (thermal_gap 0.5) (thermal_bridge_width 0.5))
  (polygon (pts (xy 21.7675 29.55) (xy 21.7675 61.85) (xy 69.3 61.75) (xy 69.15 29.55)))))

